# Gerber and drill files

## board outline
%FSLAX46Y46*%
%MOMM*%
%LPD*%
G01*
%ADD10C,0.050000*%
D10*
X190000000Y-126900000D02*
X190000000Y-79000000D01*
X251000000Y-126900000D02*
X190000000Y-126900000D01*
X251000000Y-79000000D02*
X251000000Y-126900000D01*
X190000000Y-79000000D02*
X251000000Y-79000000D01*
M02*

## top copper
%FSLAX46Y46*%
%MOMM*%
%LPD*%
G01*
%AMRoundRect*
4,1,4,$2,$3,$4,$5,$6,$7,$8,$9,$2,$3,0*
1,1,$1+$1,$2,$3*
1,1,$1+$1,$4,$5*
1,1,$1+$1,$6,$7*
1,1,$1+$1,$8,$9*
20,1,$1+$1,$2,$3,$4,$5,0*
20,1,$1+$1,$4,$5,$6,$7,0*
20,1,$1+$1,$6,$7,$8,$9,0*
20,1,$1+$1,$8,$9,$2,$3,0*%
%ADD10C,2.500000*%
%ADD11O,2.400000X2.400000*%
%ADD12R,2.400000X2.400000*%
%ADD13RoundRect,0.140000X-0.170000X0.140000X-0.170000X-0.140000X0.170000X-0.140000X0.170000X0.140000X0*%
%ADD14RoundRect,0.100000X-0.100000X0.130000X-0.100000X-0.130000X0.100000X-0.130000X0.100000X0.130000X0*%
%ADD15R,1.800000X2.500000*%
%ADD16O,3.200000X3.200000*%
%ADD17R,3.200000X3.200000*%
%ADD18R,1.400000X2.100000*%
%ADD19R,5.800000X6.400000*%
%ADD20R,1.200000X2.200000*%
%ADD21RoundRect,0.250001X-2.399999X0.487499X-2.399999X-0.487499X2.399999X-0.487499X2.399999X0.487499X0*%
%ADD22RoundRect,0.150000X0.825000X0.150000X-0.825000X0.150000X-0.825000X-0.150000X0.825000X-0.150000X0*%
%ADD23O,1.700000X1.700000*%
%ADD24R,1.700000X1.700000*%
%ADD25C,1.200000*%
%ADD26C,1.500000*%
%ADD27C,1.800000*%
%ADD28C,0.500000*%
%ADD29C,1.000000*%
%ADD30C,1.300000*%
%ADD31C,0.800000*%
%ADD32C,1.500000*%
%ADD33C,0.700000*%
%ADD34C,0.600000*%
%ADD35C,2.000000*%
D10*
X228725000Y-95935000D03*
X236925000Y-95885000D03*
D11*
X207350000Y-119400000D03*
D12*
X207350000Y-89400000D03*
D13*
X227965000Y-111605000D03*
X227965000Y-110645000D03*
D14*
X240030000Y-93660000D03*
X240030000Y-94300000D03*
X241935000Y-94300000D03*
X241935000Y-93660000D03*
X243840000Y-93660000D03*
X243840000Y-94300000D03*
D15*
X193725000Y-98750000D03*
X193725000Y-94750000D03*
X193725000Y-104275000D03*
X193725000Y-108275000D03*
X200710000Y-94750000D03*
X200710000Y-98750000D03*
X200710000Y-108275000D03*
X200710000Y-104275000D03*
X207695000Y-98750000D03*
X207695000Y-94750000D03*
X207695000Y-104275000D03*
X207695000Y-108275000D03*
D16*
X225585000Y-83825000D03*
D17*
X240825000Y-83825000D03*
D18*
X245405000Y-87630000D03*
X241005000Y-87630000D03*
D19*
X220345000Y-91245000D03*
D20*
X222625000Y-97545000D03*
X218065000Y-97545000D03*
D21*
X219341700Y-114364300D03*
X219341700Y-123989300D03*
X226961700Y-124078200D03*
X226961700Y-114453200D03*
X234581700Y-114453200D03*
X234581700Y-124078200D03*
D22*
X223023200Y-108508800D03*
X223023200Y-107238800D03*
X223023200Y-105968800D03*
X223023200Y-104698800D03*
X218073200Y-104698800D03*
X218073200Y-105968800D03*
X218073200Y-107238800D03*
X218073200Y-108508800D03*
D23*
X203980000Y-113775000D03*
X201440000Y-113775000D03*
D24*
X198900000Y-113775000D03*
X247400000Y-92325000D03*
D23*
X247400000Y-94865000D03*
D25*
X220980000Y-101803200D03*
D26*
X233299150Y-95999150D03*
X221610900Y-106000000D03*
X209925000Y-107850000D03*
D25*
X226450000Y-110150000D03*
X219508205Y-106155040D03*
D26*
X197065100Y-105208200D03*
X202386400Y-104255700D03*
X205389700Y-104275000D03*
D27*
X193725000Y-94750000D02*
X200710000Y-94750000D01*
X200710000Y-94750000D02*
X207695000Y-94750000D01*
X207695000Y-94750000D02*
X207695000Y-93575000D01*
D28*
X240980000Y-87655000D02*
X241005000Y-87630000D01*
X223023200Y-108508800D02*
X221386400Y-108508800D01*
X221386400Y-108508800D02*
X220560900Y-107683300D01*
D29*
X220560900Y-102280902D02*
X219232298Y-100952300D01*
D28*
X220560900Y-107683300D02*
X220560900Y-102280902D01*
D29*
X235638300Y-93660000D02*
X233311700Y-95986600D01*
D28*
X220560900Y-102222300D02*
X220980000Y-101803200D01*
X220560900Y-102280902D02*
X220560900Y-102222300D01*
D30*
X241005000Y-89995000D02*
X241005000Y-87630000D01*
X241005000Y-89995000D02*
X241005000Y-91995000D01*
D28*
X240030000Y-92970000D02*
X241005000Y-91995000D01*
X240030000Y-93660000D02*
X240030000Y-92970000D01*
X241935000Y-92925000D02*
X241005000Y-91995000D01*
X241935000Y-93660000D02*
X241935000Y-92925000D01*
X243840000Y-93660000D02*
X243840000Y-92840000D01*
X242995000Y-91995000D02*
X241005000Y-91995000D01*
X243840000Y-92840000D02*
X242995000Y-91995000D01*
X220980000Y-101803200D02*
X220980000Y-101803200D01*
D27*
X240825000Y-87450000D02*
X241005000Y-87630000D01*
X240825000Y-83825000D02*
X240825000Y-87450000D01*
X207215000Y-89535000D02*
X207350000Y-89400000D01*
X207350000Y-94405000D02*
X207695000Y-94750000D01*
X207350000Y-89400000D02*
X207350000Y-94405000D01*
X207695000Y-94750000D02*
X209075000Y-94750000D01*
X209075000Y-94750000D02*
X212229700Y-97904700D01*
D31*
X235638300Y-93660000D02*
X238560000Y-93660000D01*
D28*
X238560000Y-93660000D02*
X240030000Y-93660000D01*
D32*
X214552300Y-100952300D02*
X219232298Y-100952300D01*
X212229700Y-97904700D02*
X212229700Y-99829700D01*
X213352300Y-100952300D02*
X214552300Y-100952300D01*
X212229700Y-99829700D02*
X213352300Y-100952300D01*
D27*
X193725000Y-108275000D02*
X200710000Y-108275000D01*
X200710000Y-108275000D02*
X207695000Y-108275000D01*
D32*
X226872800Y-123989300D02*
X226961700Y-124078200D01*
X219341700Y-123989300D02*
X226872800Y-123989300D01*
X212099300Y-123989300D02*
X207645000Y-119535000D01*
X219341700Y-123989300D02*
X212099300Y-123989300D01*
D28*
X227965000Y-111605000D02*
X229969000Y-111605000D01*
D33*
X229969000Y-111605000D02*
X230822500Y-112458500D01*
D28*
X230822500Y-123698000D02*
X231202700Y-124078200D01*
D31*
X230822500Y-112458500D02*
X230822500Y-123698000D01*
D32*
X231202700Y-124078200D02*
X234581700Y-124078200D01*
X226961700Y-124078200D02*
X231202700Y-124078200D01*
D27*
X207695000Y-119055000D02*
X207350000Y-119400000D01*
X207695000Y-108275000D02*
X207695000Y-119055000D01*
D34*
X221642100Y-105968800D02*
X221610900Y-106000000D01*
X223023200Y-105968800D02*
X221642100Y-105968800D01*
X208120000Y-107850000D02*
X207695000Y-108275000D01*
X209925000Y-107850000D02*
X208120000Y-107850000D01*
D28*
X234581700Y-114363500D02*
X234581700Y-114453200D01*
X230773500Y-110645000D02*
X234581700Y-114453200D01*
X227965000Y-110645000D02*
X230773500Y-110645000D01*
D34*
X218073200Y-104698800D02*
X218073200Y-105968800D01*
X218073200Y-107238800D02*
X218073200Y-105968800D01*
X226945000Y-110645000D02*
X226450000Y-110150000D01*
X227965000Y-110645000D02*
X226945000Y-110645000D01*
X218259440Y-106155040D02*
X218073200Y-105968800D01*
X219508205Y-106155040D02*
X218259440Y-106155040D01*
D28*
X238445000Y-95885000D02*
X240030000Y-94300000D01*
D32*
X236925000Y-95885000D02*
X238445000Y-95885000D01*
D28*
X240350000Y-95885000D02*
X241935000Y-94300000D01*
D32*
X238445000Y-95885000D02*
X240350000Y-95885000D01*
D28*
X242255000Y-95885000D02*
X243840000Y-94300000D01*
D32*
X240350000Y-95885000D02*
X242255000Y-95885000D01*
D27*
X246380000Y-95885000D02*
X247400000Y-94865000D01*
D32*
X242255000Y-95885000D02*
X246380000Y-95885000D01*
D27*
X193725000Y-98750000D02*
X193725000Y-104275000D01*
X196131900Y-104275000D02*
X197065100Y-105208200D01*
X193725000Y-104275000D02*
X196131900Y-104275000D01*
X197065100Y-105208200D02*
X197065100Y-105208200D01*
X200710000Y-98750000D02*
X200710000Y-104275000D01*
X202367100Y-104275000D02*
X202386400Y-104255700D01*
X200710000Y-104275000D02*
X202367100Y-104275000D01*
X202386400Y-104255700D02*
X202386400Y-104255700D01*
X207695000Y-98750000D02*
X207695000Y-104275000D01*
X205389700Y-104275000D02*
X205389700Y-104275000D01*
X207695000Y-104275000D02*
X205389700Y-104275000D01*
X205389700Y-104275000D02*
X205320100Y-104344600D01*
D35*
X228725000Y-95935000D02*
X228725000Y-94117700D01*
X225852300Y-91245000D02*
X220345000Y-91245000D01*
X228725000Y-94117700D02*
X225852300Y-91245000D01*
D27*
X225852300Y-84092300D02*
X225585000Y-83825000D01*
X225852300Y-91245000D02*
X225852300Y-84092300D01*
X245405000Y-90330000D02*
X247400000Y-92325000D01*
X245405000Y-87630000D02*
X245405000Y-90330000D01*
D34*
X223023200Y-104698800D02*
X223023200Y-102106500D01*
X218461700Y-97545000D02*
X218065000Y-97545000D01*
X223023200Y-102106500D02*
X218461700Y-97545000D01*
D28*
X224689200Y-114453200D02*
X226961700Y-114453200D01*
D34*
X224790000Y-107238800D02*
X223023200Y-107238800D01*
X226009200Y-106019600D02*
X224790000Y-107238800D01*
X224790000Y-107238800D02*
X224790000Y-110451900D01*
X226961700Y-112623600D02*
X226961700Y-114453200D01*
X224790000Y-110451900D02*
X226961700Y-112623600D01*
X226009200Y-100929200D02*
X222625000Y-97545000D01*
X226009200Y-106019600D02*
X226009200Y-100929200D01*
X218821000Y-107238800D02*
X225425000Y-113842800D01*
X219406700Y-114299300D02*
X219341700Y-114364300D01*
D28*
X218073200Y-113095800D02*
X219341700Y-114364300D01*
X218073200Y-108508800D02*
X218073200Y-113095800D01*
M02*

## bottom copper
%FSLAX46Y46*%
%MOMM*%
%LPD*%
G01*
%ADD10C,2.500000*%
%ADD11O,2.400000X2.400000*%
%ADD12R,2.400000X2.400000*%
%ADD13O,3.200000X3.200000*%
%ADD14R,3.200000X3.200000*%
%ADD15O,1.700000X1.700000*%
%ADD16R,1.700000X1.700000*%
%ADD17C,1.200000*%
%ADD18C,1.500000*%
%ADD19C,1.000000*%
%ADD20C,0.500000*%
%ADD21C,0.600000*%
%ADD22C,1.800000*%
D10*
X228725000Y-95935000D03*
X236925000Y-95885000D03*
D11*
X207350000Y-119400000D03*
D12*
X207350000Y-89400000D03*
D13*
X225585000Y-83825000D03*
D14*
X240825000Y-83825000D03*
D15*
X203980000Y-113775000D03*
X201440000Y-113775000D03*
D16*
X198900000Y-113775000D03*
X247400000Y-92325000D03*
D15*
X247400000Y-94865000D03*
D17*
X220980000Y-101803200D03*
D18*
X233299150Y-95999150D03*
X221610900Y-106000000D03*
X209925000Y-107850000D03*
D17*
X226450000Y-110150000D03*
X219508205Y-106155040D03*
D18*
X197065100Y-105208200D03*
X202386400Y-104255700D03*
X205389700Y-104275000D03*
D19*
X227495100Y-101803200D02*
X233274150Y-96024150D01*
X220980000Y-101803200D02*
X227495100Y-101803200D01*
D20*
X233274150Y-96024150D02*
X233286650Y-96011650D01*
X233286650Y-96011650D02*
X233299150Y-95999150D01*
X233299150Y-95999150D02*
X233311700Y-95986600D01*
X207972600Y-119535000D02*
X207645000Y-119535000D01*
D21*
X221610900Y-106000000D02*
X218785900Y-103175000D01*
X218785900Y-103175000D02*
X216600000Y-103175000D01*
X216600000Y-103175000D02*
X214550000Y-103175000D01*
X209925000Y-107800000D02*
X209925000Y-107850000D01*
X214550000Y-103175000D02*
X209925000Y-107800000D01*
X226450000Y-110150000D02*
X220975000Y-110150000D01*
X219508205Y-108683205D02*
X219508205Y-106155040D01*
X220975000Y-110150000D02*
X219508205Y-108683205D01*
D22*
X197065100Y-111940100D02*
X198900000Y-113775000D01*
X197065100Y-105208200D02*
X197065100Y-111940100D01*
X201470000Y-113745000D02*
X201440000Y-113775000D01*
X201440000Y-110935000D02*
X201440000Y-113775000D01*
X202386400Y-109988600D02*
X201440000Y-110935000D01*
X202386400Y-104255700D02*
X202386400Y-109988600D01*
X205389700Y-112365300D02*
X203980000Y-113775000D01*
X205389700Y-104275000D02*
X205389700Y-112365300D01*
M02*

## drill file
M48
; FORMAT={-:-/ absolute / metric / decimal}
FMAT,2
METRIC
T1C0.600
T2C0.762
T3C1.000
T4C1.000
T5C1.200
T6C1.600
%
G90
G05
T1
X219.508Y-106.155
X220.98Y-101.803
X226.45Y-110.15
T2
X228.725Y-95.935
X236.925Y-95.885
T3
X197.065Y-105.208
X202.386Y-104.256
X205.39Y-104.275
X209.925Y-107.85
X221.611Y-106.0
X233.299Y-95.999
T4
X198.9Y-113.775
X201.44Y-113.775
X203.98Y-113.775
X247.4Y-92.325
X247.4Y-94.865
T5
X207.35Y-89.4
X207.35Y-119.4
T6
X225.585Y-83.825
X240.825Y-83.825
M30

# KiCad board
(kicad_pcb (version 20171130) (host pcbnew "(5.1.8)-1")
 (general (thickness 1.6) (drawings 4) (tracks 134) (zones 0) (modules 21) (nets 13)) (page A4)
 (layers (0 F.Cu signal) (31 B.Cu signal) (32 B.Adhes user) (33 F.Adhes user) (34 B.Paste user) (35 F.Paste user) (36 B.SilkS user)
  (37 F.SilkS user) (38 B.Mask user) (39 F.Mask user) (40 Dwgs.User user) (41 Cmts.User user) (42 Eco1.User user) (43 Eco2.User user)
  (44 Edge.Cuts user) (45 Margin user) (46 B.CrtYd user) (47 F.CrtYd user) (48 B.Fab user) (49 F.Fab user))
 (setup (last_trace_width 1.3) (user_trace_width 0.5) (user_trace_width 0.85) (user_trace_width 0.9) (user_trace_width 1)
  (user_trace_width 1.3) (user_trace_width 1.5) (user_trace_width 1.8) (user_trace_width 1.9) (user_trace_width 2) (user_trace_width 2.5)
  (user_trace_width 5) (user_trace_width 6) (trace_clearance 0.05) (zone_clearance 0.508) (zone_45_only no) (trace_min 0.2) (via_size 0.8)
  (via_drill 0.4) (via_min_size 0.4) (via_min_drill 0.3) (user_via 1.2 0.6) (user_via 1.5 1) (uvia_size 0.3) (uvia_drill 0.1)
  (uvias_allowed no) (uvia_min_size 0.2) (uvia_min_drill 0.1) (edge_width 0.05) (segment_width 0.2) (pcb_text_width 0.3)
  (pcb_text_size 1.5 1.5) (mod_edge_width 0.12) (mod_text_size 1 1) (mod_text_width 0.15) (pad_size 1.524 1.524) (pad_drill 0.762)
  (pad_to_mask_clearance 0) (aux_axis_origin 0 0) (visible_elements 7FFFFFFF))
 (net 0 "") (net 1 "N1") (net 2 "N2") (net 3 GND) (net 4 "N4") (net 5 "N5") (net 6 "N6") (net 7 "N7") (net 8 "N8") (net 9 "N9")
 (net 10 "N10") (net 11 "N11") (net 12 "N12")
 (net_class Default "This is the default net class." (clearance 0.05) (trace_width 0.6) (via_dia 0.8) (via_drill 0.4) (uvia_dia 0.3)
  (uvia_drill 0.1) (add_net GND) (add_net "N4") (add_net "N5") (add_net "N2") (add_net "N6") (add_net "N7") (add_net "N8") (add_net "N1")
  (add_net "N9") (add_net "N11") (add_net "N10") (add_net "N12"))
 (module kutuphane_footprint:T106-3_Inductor (layer F.Cu) (at 231.775 95.885 90)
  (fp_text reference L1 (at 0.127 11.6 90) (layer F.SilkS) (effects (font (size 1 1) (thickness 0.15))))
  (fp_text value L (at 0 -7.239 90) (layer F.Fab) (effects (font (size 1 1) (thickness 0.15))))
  (pad 1 thru_hole circle (at -0.05 -3.05 90) (size 2.5 2.5) (drill 0.762) (layers *.Cu *.Mask) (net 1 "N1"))
  (pad 2 thru_hole circle (at 0 5.15 90) (size 2.5 2.5) (drill 0.762) (layers *.Cu *.Mask) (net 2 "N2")))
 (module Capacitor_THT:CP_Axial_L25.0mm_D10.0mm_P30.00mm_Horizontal (layer B.Cu) (at 207.35 89.4 270)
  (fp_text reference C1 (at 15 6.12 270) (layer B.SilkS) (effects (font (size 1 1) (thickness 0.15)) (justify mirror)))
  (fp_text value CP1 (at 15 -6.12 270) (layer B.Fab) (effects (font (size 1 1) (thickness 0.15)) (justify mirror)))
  (pad 2 thru_hole oval (at 30 0 270) (size 2.4 2.4) (drill 1.2) (layers *.Cu *.Mask) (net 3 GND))
  (pad 1 thru_hole rect (at 0 0 270) (size 2.4 2.4) (drill 1.2) (layers *.Cu *.Mask) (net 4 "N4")))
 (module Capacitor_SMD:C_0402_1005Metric (layer F.Cu) (at 227.965 111.125 270)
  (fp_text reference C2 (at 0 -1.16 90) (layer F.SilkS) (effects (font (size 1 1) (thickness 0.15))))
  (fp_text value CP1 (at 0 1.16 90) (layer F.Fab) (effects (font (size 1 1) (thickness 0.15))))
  (pad 2 smd roundrect (at 0.48 0 270) (size 0.56 0.62) (layers F.Cu F.Paste F.Mask) (roundrect_rratio 0.25) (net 3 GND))
  (pad 1 smd roundrect (at -0.48 0 270) (size 0.56 0.62) (layers F.Cu F.Paste F.Mask) (roundrect_rratio 0.25) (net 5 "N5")))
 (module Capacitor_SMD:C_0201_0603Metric (layer F.Cu) (at 240.03 93.98 270)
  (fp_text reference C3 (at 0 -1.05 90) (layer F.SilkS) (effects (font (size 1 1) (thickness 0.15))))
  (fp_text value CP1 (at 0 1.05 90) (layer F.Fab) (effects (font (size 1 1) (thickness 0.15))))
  (pad "" smd roundrect (at -0.345 0 270) (size 0.318 0.36) (layers F.Paste) (roundrect_rratio 0.25))
  (pad "" smd roundrect (at 0.345 0 270) (size 0.318 0.36) (layers F.Paste) (roundrect_rratio 0.25))
  (pad 1 smd roundrect (at -0.32 0 270) (size 0.46 0.4) (layers F.Cu F.Mask) (roundrect_rratio 0.25) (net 4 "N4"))
  (pad 2 smd roundrect (at 0.32 0 270) (size 0.46 0.4) (layers F.Cu F.Mask) (roundrect_rratio 0.25) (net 2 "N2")))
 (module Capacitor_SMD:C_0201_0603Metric (layer F.Cu) (at 241.935 93.98 270)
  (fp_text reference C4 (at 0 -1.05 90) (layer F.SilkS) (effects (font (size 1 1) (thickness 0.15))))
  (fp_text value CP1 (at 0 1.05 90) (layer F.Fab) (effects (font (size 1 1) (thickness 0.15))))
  (pad 2 smd roundrect (at 0.32 0 270) (size 0.46 0.4) (layers F.Cu F.Mask) (roundrect_rratio 0.25) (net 2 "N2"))
  (pad 1 smd roundrect (at -0.32 0 270) (size 0.46 0.4) (layers F.Cu F.Mask) (roundrect_rratio 0.25) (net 4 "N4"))
  (pad "" smd roundrect (at 0.345 0 270) (size 0.318 0.36) (layers F.Paste) (roundrect_rratio 0.25))
  (pad "" smd roundrect (at -0.345 0 270) (size 0.318 0.36) (layers F.Paste) (roundrect_rratio 0.25)))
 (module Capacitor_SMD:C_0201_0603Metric (layer F.Cu) (at 243.84 93.98 270)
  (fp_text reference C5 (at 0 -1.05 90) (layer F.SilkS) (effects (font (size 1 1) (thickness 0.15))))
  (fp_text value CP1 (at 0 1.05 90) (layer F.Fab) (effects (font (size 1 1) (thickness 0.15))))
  (pad "" smd roundrect (at -0.345 0 270) (size 0.318 0.36) (layers F.Paste) (roundrect_rratio 0.25))
  (pad "" smd roundrect (at 0.345 0 270) (size 0.318 0.36) (layers F.Paste) (roundrect_rratio 0.25))
  (pad 1 smd roundrect (at -0.32 0 270) (size 0.46 0.4) (layers F.Cu F.Mask) (roundrect_rratio 0.25) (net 4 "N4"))
  (pad 2 smd roundrect (at 0.32 0 270) (size 0.46 0.4) (layers F.Cu F.Mask) (roundrect_rratio 0.25) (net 2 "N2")))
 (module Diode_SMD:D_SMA (layer F.Cu) (at 193.725 96.75 270)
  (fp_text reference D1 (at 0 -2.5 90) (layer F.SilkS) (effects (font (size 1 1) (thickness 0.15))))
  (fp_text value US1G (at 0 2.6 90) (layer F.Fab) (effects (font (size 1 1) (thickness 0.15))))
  (pad 2 smd rect (at 2 0 270) (size 2.5 1.8) (layers F.Cu F.Paste F.Mask) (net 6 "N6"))
  (pad 1 smd rect (at -2 0 270) (size 2.5 1.8) (layers F.Cu F.Paste F.Mask) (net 4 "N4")))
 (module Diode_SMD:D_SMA (layer F.Cu) (at 193.725 106.275 270)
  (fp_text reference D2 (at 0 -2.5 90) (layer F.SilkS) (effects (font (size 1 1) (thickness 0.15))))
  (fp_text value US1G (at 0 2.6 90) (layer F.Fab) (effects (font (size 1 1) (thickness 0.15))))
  (pad 1 smd rect (at -2 0 270) (size 2.5 1.8) (layers F.Cu F.Paste F.Mask) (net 6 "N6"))
  (pad 2 smd rect (at 2 0 270) (size 2.5 1.8) (layers F.Cu F.Paste F.Mask) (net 3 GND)))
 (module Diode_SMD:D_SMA (layer F.Cu) (at 200.71 96.75 270)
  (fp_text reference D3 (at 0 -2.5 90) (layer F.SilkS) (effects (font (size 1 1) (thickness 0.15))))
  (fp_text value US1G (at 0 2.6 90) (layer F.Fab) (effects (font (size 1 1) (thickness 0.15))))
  (pad 1 smd rect (at -2 0 270) (size 2.5 1.8) (layers F.Cu F.Paste F.Mask) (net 4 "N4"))
  (pad 2 smd rect (at 2 0 270) (size 2.5 1.8) (layers F.Cu F.Paste F.Mask) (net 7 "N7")))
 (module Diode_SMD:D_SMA (layer F.Cu) (at 200.71 106.275 270)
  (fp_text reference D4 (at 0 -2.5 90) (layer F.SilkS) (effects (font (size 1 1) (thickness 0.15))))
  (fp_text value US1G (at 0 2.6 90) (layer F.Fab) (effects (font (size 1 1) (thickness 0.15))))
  (pad 2 smd rect (at 2 0 270) (size 2.5 1.8) (layers F.Cu F.Paste F.Mask) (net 3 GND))
  (pad 1 smd rect (at -2 0 270) (size 2.5 1.8) (layers F.Cu F.Paste F.Mask) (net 7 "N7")))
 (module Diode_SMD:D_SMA (layer F.Cu) (at 207.695 96.75 270)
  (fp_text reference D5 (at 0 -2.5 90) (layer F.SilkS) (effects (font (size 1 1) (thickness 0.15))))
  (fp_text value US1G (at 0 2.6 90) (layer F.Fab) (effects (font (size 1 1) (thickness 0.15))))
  (pad 2 smd rect (at 2 0 270) (size 2.5 1.8) (layers F.Cu F.Paste F.Mask) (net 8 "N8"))
  (pad 1 smd rect (at -2 0 270) (size 2.5 1.8) (layers F.Cu F.Paste F.Mask) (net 4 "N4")))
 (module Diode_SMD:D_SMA (layer F.Cu) (at 207.695 106.275 270)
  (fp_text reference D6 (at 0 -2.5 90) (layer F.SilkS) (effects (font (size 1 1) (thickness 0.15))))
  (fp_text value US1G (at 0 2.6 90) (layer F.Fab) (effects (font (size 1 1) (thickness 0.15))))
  (pad 1 smd rect (at -2 0 270) (size 2.5 1.8) (layers F.Cu F.Paste F.Mask) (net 8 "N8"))
  (pad 2 smd rect (at 2 0 270) (size 2.5 1.8) (layers F.Cu F.Paste F.Mask) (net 3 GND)))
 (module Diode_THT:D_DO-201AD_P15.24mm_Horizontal (layer B.Cu) (at 240.825 83.825 180)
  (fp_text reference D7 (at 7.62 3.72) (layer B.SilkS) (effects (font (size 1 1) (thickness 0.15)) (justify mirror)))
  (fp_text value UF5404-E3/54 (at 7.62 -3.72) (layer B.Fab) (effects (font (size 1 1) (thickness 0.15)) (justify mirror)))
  (pad 2 thru_hole oval (at 15.24 0 180) (size 3.2 3.2) (drill 1.6) (layers *.Cu *.Mask) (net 1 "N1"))
  (pad 1 thru_hole rect (at 0 0 180) (size 3.2 3.2) (drill 1.6) (layers *.Cu *.Mask) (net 4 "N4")))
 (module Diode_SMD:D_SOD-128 (layer F.Cu) (at 243.205 87.63 180)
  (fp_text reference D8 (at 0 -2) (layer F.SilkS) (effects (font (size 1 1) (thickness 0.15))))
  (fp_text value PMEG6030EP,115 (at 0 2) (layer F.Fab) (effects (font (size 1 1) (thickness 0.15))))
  (pad 1 smd rect (at -2.2 0 180) (size 1.4 2.1) (layers F.Cu F.Paste F.Mask) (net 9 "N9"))
  (pad 2 smd rect (at 2.2 0 180) (size 1.4 2.1) (layers F.Cu F.Paste F.Mask) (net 4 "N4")))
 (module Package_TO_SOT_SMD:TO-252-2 (layer F.Cu) (at 220.345 93.345 90)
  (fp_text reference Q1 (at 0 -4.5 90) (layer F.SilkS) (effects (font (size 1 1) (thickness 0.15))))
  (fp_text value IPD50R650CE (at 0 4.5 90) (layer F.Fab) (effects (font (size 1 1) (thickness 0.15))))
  (pad "" smd rect (at 0.425 1.525 90) (size 3.05 2.75) (layers F.Paste))
  (pad "" smd rect (at 3.775 -1.525 90) (size 3.05 2.75) (layers F.Paste))
  (pad "" smd rect (at 0.425 -1.525 90) (size 3.05 2.75) (layers F.Paste))
  (pad "" smd rect (at 3.775 1.525 90) (size 3.05 2.75) (layers F.Paste))
  (pad 2 smd rect (at 2.1 0 90) (size 6.4 5.8) (layers F.Cu F.Mask) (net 1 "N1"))
  (pad 3 smd rect (at -4.2 2.28 90) (size 2.2 1.2) (layers F.Cu F.Paste F.Mask) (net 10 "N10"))
  (pad 1 smd rect (at -4.2 -2.28 90) (size 2.2 1.2) (layers F.Cu F.Paste F.Mask) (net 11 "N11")))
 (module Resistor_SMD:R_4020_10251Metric (layer F.Cu) (at 219.3417 119.1768 270)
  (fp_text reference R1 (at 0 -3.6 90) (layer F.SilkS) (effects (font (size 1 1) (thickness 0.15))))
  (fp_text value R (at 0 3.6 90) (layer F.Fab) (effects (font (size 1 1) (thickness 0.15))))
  (pad 1 smd roundrect (at -4.8125 0 270) (size 1.475 5.3) (layers F.Cu F.Paste F.Mask) (roundrect_rratio 0.169492) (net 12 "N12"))
  (pad 2 smd roundrect (at 4.8125 0 270) (size 1.475 5.3) (layers F.Cu F.Paste F.Mask) (roundrect_rratio 0.169492) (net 3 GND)))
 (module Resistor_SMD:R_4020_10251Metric (layer F.Cu) (at 226.9617 119.2657 270)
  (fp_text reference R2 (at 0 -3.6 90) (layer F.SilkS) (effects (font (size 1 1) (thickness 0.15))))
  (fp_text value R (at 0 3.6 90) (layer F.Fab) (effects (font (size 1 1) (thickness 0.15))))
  (pad 2 smd roundrect (at 4.8125 0 270) (size 1.475 5.3) (layers F.Cu F.Paste F.Mask) (roundrect_rratio 0.169492) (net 3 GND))
  (pad 1 smd roundrect (at -4.8125 0 270) (size 1.475 5.3) (layers F.Cu F.Paste F.Mask) (roundrect_rratio 0.169492) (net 10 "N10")))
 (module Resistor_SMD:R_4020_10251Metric (layer F.Cu) (at 234.5817 119.2657 270)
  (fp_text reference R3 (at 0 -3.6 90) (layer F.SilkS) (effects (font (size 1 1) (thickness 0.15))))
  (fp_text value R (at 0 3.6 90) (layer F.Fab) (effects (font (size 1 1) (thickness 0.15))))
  (pad 1 smd roundrect (at -4.8125 0 270) (size 1.475 5.3) (layers F.Cu F.Paste F.Mask) (roundrect_rratio 0.169492) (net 5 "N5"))
  (pad 2 smd roundrect (at 4.8125 0 270) (size 1.475 5.3) (layers F.Cu F.Paste F.Mask) (roundrect_rratio 0.169492) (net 3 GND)))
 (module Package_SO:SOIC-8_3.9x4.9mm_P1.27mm (layer F.Cu) (at 220.5482 106.6038 180)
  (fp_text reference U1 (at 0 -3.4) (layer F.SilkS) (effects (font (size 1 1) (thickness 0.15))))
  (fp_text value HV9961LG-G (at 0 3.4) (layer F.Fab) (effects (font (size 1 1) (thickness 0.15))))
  (pad 1 smd roundrect (at -2.475 -1.905 180) (size 1.95 0.6) (layers F.Cu F.Paste F.Mask) (roundrect_rratio 0.25) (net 4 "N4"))
  (pad 2 smd roundrect (at -2.475 -0.635 180) (size 1.95 0.6) (layers F.Cu F.Paste F.Mask) (roundrect_rratio 0.25) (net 10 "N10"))
  (pad 3 smd roundrect (at -2.475 0.635 180) (size 1.95 0.6) (layers F.Cu F.Paste F.Mask) (roundrect_rratio 0.25) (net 3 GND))
  (pad 4 smd roundrect (at -2.475 1.905 180) (size 1.95 0.6) (layers F.Cu F.Paste F.Mask) (roundrect_rratio 0.25) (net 11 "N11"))
  (pad 5 smd roundrect (at 2.475 1.905 180) (size 1.95 0.6) (layers F.Cu F.Paste F.Mask) (roundrect_rratio 0.25) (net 5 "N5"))
  (pad 6 smd roundrect (at 2.475 0.635 180) (size 1.95 0.6) (layers F.Cu F.Paste F.Mask) (roundrect_rratio 0.25) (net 5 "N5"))
  (pad 7 smd roundrect (at 2.475 -0.635 180) (size 1.95 0.6) (layers F.Cu F.Paste F.Mask) (roundrect_rratio 0.25) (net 5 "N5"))
  (pad 8 smd roundrect (at 2.475 -1.905 180) (size 1.95 0.6) (layers F.Cu F.Paste F.Mask) (roundrect_rratio 0.25) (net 12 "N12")))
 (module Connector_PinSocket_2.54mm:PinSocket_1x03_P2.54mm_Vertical (layer F.Cu) (at 198.9 113.775 90)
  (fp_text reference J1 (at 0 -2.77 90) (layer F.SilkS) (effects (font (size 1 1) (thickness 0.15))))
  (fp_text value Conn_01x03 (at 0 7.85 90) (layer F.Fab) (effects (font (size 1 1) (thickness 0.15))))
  (pad 3 thru_hole oval (at 0 5.08 90) (size 1.7 1.7) (drill 1) (layers *.Cu *.Mask) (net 8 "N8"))
  (pad 2 thru_hole oval (at 0 2.54 90) (size 1.7 1.7) (drill 1) (layers *.Cu *.Mask) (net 7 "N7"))
  (pad 1 thru_hole rect (at 0 0 90) (size 1.7 1.7) (drill 1) (layers *.Cu *.Mask) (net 6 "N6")))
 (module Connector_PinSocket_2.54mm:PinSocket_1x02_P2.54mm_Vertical (layer F.Cu) (at 247.4 92.325)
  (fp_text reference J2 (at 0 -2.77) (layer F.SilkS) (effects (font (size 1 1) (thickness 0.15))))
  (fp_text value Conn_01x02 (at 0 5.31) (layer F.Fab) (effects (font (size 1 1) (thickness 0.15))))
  (pad 1 thru_hole rect (at 0 0) (size 1.7 1.7) (drill 1) (layers *.Cu *.Mask) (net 9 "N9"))
  (pad 2 thru_hole oval (at 0 2.54) (size 1.7 1.7) (drill 1) (layers *.Cu *.Mask) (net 2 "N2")))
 (gr_line (start 190 126.9) (end 190 79) (layer Edge.Cuts) (width 0.05))
 (gr_line (start 251 126.9) (end 190 126.9) (layer Edge.Cuts) (width 0.05))
 (gr_line (start 251 79) (end 251 126.9) (layer Edge.Cuts) (width 0.05))
 (gr_line (start 190 79) (end 251 79) (layer Edge.Cuts) (width 0.05))
 (segment (start 193.725 94.75) (end 200.71 94.75) (width 1.8) (layer F.Cu) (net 4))
 (segment (start 200.71 94.75) (end 207.695 94.75) (width 1.8) (layer F.Cu) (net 4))
 (segment (start 207.695 94.75) (end 207.695 93.575) (width 1.8) (layer F.Cu) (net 4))
 (segment (start 240.98 87.655) (end 241.005 87.63) (width 0.5) (layer F.Cu) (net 4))
 (segment (start 223.0232 108.5088) (end 221.3864 108.5088) (width 0.5) (layer F.Cu) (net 4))
 (segment (start 221.3864 108.5088) (end 220.5609 107.6833) (width 0.5) (layer F.Cu) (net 4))
 (segment (start 220.5609 102.280902) (end 219.232298 100.9523) (width 1) (layer F.Cu) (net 4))
 (segment (start 220.5609 107.6833) (end 220.5609 102.280902) (width 0.5) (layer F.Cu) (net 4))
 (segment (start 235.6383 93.66) (end 233.3117 95.9866) (width 1) (layer F.Cu) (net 4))
 (segment (start 220.5609 102.2223) (end 220.98 101.8032) (width 0.5) (layer F.Cu) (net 4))
 (segment (start 220.5609 102.280902) (end 220.5609 102.2223) (width 0.5) (layer F.Cu) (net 4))
 (segment (start 227.4951 101.8032) (end 233.27415 96.02415) (width 1) (layer B.Cu) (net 4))
 (segment (start 220.98 101.8032) (end 227.4951 101.8032) (width 1) (layer B.Cu) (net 4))
 (segment (start 241.005 89.995) (end 241.005 87.63) (width 1.3) (layer F.Cu) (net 4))
 (segment (start 241.005 89.995) (end 241.005 91.995) (width 1.3) (layer F.Cu) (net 4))
 (segment (start 240.03 92.97) (end 241.005 91.995) (width 0.5) (layer F.Cu) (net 4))
 (segment (start 240.03 93.66) (end 240.03 92.97) (width 0.5) (layer F.Cu) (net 4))
 (segment (start 241.935 92.925) (end 241.005 91.995) (width 0.5) (layer F.Cu) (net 4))
 (segment (start 241.935 93.66) (end 241.935 92.925) (width 0.5) (layer F.Cu) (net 4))
 (segment (start 243.84 93.66) (end 243.84 92.84) (width 0.5) (layer F.Cu) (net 4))
 (segment (start 242.995 91.995) (end 241.005 91.995) (width 0.5) (layer F.Cu) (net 4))
 (segment (start 243.84 92.84) (end 242.995 91.995) (width 0.5) (layer F.Cu) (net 4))
 (segment (start 233.27415 96.02415) (end 233.28665 96.01165) (width 0.5) (layer B.Cu) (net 4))
 (segment (start 233.28665 96.01165) (end 233.29915 95.99915) (width 0.5) (layer B.Cu) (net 4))
 (segment (start 220.98 101.8032) (end 220.98 101.8032) (width 0.5) (layer F.Cu) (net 4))
 (via (at 220.98 101.8032) (size 1.2) (drill 0.6) (layers F.Cu B.Cu) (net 4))
 (segment (start 233.29915 95.99915) (end 233.3117 95.9866) (width 0.5) (layer B.Cu) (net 4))
 (via (at 233.29915 95.99915) (size 1.5) (drill 1) (layers F.Cu B.Cu) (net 4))
 (segment (start 240.825 87.45) (end 241.005 87.63) (width 1.8) (layer F.Cu) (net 4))
 (segment (start 240.825 83.825) (end 240.825 87.45) (width 1.8) (layer F.Cu) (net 4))
 (segment (start 207.215 89.535) (end 207.35 89.4) (width 1.8) (layer F.Cu) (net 4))
 (segment (start 207.35 94.405) (end 207.695 94.75) (width 1.8) (layer F.Cu) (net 4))
 (segment (start 207.35 89.4) (end 207.35 94.405) (width 1.8) (layer F.Cu) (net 4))
 (segment (start 207.695 94.75) (end 209.075 94.75) (width 1.8) (layer F.Cu) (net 4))
 (segment (start 209.075 94.75) (end 212.2297 97.9047) (width 1.8) (layer F.Cu) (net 4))
 (segment (start 235.6383 93.66) (end 238.56 93.66) (width 0.8) (layer F.Cu) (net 4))
 (segment (start 238.56 93.66) (end 240.03 93.66) (width 0.5) (layer F.Cu) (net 4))
 (segment (start 214.5523 100.9523) (end 219.232298 100.9523) (width 1.5) (layer F.Cu) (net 4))
 (segment (start 212.2297 97.9047) (end 212.2297 99.8297) (width 1.5) (layer F.Cu) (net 4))
 (segment (start 213.3523 100.9523) (end 214.5523 100.9523) (width 1.5) (layer F.Cu) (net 4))
 (segment (start 212.2297 99.8297) (end 213.3523 100.9523) (width 1.5) (layer F.Cu) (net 4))
 (segment (start 193.725 108.275) (end 200.71 108.275) (width 1.8) (layer F.Cu) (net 3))
 (segment (start 200.71 108.275) (end 207.695 108.275) (width 1.8) (layer F.Cu) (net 3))
 (segment (start 207.9726 119.535) (end 207.645 119.535) (width 0.5) (layer B.Cu) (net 3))
 (segment (start 226.8728 123.9893) (end 226.9617 124.0782) (width 1.5) (layer F.Cu) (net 3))
 (segment (start 219.3417 123.9893) (end 226.8728 123.9893) (width 1.5) (layer F.Cu) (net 3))
 (segment (start 212.0993 123.9893) (end 207.645 119.535) (width 1.5) (layer F.Cu) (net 3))
 (segment (start 219.3417 123.9893) (end 212.0993 123.9893) (width 1.5) (layer F.Cu) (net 3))
 (segment (start 227.965 111.605) (end 229.969 111.605) (width 0.5) (layer F.Cu) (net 3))
 (segment (start 229.969 111.605) (end 230.8225 112.4585) (width 0.7) (layer F.Cu) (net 3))
 (segment (start 230.8225 123.698) (end 231.2027 124.0782) (width 0.5) (layer F.Cu) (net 3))
 (segment (start 230.8225 112.4585) (end 230.8225 123.698) (width 0.8) (layer F.Cu) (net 3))
 (segment (start 231.2027 124.0782) (end 234.5817 124.0782) (width 1.5) (layer F.Cu) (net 3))
 (segment (start 226.9617 124.0782) (end 231.2027 124.0782) (width 1.5) (layer F.Cu) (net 3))
 (segment (start 207.695 119.055) (end 207.35 119.4) (width 1.8) (layer F.Cu) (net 3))
 (segment (start 207.695 108.275) (end 207.695 119.055) (width 1.8) (layer F.Cu) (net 3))
 (via (at 221.6109 106) (size 1.5) (drill 1) (layers F.Cu B.Cu) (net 3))
 (segment (start 221.6421 105.9688) (end 221.6109 106) (width 0.6) (layer F.Cu) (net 3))
 (segment (start 223.0232 105.9688) (end 221.6421 105.9688) (width 0.6) (layer F.Cu) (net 3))
 (segment (start 221.6109 106) (end 218.7859 103.175) (width 0.6) (layer B.Cu) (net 3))
 (segment (start 218.7859 103.175) (end 216.6 103.175) (width 0.6) (layer B.Cu) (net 3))
 (segment (start 216.6 103.175) (end 214.55 103.175) (width 0.6) (layer B.Cu) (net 3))
 (via (at 209.925 107.85) (size 1.5) (drill 1) (layers F.Cu B.Cu) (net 3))
 (segment (start 209.925 107.8) (end 209.925 107.85) (width 0.6) (layer B.Cu) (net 3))
 (segment (start 214.55 103.175) (end 209.925 107.8) (width 0.6) (layer B.Cu) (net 3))
 (segment (start 208.12 107.85) (end 207.695 108.275) (width 0.6) (layer F.Cu) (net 3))
 (segment (start 209.925 107.85) (end 208.12 107.85) (width 0.6) (layer F.Cu) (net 3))
 (segment (start 234.5817 114.3635) (end 234.5817 114.4532) (width 0.5) (layer F.Cu) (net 5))
 (segment (start 230.7735 110.645) (end 234.5817 114.4532) (width 0.5) (layer F.Cu) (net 5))
 (segment (start 227.965 110.645) (end 230.7735 110.645) (width 0.5) (layer F.Cu) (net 5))
 (segment (start 218.0732 104.6988) (end 218.0732 105.9688) (width 0.6) (layer F.Cu) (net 5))
 (segment (start 218.0732 107.2388) (end 218.0732 105.9688) (width 0.6) (layer F.Cu) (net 5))
 (via (at 226.45 110.15) (size 1.2) (drill 0.6) (layers F.Cu B.Cu) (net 5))
 (segment (start 226.945 110.645) (end 226.45 110.15) (width 0.6) (layer F.Cu) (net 5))
 (segment (start 227.965 110.645) (end 226.945 110.645) (width 0.6) (layer F.Cu) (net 5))
 (segment (start 226.45 110.15) (end 220.975 110.15) (width 0.6) (layer B.Cu) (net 5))
 (via (at 219.508205 106.15504) (size 1.2) (drill 0.6) (layers F.Cu B.Cu) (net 5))
 (segment (start 219.508205 108.683205) (end 219.508205 106.15504) (width 0.6) (layer B.Cu) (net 5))
 (segment (start 220.975 110.15) (end 219.508205 108.683205) (width 0.6) (layer B.Cu) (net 5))
 (segment (start 218.25944 106.15504) (end 218.0732 105.9688) (width 0.6) (layer F.Cu) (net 5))
 (segment (start 219.508205 106.15504) (end 218.25944 106.15504) (width 0.6) (layer F.Cu) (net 5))
 (segment (start 238.445 95.885) (end 240.03 94.3) (width 0.5) (layer F.Cu) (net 2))
 (segment (start 236.925 95.885) (end 238.445 95.885) (width 1.5) (layer F.Cu) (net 2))
 (segment (start 240.35 95.885) (end 241.935 94.3) (width 0.5) (layer F.Cu) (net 2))
 (segment (start 238.445 95.885) (end 240.35 95.885) (width 1.5) (layer F.Cu) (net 2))
 (segment (start 242.255 95.885) (end 243.84 94.3) (width 0.5) (layer F.Cu) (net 2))
 (segment (start 240.35 95.885) (end 242.255 95.885) (width 1.5) (layer F.Cu) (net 2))
 (segment (start 246.38 95.885) (end 247.4 94.865) (width 1.8) (layer F.Cu) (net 2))
 (segment (start 242.255 95.885) (end 246.38 95.885) (width 1.5) (layer F.Cu) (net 2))
 (segment (start 193.725 98.75) (end 193.725 104.275) (width 1.8) (layer F.Cu) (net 6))
 (segment (start 196.1319 104.275) (end 197.0651 105.2082) (width 1.8) (layer F.Cu) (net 6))
 (segment (start 193.725 104.275) (end 196.1319 104.275) (width 1.8) (layer F.Cu) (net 6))
 (segment (start 197.0651 105.2082) (end 197.0651 105.2082) (width 1.8) (layer F.Cu) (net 6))
 (via (at 197.0651 105.2082) (size 1.5) (drill 1) (layers F.Cu B.Cu) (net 6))
 (segment (start 197.0651 111.9401) (end 198.9 113.775) (width 1.8) (layer B.Cu) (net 6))
 (segment (start 197.0651 105.2082) (end 197.0651 111.9401) (width 1.8) (layer B.Cu) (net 6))
 (segment (start 200.71 98.75) (end 200.71 104.275) (width 1.8) (layer F.Cu) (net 7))
 (segment (start 202.3671 104.275) (end 202.3864 104.2557) (width 1.8) (layer F.Cu) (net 7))
 (segment (start 200.71 104.275) (end 202.3671 104.275) (width 1.8) (layer F.Cu) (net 7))
 (segment (start 202.3864 104.2557) (end 202.3864 104.2557) (width 1.8) (layer F.Cu) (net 7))
 (via (at 202.3864 104.2557) (size 1.5) (drill 1) (layers F.Cu B.Cu) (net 7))
 (segment (start 201.47 113.745) (end 201.44 113.775) (width 1.8) (layer B.Cu) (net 7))
 (segment (start 201.44 110.935) (end 201.44 113.775) (width 1.8) (layer B.Cu) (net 7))
 (segment (start 202.3864 109.9886) (end 201.44 110.935) (width 1.8) (layer B.Cu) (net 7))
 (segment (start 202.3864 104.2557) (end 202.3864 109.9886) (width 1.8) (layer B.Cu) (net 7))
 (segment (start 207.695 98.75) (end 207.695 104.275) (width 1.8) (layer F.Cu) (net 8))
 (segment (start 205.3897 104.275) (end 205.3897 104.275) (width 1.8) (layer F.Cu) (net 8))
 (segment (start 207.695 104.275) (end 205.3897 104.275) (width 1.8) (layer F.Cu) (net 8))
 (segment (start 205.3897 104.275) (end 205.3201 104.3446) (width 1.8) (layer F.Cu) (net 8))
 (via (at 205.3897 104.275) (size 1.5) (drill 1) (layers F.Cu B.Cu) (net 8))
 (segment (start 205.3897 112.3653) (end 203.98 113.775) (width 1.8) (layer B.Cu) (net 8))
 (segment (start 205.3897 104.275) (end 205.3897 112.3653) (width 1.8) (layer B.Cu) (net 8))
 (segment (start 228.725 95.935) (end 228.725 94.1177) (width 2) (layer F.Cu) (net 1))
 (segment (start 225.8523 91.245) (end 220.345 91.245) (width 2) (layer F.Cu) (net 1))
 (segment (start 228.725 94.1177) (end 225.8523 91.245) (width 2) (layer F.Cu) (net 1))
 (segment (start 225.8523 84.0923) (end 225.585 83.825) (width 1.8) (layer F.Cu) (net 1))
 (segment (start 225.8523 91.245) (end 225.8523 84.0923) (width 1.8) (layer F.Cu) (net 1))
 (segment (start 245.405 90.33) (end 247.4 92.325) (width 1.8) (layer F.Cu) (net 9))
 (segment (start 245.405 87.63) (end 245.405 90.33) (width 1.8) (layer F.Cu) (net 9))
 (segment (start 223.0232 104.6988) (end 223.0232 102.1065) (width 0.6) (layer F.Cu) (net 11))
 (segment (start 218.4617 97.545) (end 218.065 97.545) (width 0.6) (layer F.Cu) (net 11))
 (segment (start 223.0232 102.1065) (end 218.4617 97.545) (width 0.6) (layer F.Cu) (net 11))
 (segment (start 224.6892 114.4532) (end 226.9617 114.4532) (width 0.5) (layer F.Cu) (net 10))
 (segment (start 224.79 107.2388) (end 223.0232 107.2388) (width 0.6) (layer F.Cu) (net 10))
 (segment (start 226.0092 106.0196) (end 224.79 107.2388) (width 0.6) (layer F.Cu) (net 10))
 (segment (start 224.79 107.2388) (end 224.79 110.4519) (width 0.6) (layer F.Cu) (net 10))
 (segment (start 226.9617 112.6236) (end 226.9617 114.4532) (width 0.6) (layer F.Cu) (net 10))
 (segment (start 224.79 110.4519) (end 226.9617 112.6236) (width 0.6) (layer F.Cu) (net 10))
 (segment (start 226.0092 100.9292) (end 222.625 97.545) (width 0.6) (layer F.Cu) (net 10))
 (segment (start 226.0092 106.0196) (end 226.0092 100.9292) (width 0.6) (layer F.Cu) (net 10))
 (segment (start 218.821 107.2388) (end 225.425 113.8428) (width 0.6) (layer F.Cu) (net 10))
 (segment (start 219.4067 114.2993) (end 219.3417 114.3643) (width 0.6) (layer F.Cu) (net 12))
 (segment (start 218.0732 113.0958) (end 219.3417 114.3643) (width 0.5) (layer F.Cu) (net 12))
 (segment (start 218.0732 108.5088) (end 218.0732 113.0958) (width 0.5) (layer F.Cu) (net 12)))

